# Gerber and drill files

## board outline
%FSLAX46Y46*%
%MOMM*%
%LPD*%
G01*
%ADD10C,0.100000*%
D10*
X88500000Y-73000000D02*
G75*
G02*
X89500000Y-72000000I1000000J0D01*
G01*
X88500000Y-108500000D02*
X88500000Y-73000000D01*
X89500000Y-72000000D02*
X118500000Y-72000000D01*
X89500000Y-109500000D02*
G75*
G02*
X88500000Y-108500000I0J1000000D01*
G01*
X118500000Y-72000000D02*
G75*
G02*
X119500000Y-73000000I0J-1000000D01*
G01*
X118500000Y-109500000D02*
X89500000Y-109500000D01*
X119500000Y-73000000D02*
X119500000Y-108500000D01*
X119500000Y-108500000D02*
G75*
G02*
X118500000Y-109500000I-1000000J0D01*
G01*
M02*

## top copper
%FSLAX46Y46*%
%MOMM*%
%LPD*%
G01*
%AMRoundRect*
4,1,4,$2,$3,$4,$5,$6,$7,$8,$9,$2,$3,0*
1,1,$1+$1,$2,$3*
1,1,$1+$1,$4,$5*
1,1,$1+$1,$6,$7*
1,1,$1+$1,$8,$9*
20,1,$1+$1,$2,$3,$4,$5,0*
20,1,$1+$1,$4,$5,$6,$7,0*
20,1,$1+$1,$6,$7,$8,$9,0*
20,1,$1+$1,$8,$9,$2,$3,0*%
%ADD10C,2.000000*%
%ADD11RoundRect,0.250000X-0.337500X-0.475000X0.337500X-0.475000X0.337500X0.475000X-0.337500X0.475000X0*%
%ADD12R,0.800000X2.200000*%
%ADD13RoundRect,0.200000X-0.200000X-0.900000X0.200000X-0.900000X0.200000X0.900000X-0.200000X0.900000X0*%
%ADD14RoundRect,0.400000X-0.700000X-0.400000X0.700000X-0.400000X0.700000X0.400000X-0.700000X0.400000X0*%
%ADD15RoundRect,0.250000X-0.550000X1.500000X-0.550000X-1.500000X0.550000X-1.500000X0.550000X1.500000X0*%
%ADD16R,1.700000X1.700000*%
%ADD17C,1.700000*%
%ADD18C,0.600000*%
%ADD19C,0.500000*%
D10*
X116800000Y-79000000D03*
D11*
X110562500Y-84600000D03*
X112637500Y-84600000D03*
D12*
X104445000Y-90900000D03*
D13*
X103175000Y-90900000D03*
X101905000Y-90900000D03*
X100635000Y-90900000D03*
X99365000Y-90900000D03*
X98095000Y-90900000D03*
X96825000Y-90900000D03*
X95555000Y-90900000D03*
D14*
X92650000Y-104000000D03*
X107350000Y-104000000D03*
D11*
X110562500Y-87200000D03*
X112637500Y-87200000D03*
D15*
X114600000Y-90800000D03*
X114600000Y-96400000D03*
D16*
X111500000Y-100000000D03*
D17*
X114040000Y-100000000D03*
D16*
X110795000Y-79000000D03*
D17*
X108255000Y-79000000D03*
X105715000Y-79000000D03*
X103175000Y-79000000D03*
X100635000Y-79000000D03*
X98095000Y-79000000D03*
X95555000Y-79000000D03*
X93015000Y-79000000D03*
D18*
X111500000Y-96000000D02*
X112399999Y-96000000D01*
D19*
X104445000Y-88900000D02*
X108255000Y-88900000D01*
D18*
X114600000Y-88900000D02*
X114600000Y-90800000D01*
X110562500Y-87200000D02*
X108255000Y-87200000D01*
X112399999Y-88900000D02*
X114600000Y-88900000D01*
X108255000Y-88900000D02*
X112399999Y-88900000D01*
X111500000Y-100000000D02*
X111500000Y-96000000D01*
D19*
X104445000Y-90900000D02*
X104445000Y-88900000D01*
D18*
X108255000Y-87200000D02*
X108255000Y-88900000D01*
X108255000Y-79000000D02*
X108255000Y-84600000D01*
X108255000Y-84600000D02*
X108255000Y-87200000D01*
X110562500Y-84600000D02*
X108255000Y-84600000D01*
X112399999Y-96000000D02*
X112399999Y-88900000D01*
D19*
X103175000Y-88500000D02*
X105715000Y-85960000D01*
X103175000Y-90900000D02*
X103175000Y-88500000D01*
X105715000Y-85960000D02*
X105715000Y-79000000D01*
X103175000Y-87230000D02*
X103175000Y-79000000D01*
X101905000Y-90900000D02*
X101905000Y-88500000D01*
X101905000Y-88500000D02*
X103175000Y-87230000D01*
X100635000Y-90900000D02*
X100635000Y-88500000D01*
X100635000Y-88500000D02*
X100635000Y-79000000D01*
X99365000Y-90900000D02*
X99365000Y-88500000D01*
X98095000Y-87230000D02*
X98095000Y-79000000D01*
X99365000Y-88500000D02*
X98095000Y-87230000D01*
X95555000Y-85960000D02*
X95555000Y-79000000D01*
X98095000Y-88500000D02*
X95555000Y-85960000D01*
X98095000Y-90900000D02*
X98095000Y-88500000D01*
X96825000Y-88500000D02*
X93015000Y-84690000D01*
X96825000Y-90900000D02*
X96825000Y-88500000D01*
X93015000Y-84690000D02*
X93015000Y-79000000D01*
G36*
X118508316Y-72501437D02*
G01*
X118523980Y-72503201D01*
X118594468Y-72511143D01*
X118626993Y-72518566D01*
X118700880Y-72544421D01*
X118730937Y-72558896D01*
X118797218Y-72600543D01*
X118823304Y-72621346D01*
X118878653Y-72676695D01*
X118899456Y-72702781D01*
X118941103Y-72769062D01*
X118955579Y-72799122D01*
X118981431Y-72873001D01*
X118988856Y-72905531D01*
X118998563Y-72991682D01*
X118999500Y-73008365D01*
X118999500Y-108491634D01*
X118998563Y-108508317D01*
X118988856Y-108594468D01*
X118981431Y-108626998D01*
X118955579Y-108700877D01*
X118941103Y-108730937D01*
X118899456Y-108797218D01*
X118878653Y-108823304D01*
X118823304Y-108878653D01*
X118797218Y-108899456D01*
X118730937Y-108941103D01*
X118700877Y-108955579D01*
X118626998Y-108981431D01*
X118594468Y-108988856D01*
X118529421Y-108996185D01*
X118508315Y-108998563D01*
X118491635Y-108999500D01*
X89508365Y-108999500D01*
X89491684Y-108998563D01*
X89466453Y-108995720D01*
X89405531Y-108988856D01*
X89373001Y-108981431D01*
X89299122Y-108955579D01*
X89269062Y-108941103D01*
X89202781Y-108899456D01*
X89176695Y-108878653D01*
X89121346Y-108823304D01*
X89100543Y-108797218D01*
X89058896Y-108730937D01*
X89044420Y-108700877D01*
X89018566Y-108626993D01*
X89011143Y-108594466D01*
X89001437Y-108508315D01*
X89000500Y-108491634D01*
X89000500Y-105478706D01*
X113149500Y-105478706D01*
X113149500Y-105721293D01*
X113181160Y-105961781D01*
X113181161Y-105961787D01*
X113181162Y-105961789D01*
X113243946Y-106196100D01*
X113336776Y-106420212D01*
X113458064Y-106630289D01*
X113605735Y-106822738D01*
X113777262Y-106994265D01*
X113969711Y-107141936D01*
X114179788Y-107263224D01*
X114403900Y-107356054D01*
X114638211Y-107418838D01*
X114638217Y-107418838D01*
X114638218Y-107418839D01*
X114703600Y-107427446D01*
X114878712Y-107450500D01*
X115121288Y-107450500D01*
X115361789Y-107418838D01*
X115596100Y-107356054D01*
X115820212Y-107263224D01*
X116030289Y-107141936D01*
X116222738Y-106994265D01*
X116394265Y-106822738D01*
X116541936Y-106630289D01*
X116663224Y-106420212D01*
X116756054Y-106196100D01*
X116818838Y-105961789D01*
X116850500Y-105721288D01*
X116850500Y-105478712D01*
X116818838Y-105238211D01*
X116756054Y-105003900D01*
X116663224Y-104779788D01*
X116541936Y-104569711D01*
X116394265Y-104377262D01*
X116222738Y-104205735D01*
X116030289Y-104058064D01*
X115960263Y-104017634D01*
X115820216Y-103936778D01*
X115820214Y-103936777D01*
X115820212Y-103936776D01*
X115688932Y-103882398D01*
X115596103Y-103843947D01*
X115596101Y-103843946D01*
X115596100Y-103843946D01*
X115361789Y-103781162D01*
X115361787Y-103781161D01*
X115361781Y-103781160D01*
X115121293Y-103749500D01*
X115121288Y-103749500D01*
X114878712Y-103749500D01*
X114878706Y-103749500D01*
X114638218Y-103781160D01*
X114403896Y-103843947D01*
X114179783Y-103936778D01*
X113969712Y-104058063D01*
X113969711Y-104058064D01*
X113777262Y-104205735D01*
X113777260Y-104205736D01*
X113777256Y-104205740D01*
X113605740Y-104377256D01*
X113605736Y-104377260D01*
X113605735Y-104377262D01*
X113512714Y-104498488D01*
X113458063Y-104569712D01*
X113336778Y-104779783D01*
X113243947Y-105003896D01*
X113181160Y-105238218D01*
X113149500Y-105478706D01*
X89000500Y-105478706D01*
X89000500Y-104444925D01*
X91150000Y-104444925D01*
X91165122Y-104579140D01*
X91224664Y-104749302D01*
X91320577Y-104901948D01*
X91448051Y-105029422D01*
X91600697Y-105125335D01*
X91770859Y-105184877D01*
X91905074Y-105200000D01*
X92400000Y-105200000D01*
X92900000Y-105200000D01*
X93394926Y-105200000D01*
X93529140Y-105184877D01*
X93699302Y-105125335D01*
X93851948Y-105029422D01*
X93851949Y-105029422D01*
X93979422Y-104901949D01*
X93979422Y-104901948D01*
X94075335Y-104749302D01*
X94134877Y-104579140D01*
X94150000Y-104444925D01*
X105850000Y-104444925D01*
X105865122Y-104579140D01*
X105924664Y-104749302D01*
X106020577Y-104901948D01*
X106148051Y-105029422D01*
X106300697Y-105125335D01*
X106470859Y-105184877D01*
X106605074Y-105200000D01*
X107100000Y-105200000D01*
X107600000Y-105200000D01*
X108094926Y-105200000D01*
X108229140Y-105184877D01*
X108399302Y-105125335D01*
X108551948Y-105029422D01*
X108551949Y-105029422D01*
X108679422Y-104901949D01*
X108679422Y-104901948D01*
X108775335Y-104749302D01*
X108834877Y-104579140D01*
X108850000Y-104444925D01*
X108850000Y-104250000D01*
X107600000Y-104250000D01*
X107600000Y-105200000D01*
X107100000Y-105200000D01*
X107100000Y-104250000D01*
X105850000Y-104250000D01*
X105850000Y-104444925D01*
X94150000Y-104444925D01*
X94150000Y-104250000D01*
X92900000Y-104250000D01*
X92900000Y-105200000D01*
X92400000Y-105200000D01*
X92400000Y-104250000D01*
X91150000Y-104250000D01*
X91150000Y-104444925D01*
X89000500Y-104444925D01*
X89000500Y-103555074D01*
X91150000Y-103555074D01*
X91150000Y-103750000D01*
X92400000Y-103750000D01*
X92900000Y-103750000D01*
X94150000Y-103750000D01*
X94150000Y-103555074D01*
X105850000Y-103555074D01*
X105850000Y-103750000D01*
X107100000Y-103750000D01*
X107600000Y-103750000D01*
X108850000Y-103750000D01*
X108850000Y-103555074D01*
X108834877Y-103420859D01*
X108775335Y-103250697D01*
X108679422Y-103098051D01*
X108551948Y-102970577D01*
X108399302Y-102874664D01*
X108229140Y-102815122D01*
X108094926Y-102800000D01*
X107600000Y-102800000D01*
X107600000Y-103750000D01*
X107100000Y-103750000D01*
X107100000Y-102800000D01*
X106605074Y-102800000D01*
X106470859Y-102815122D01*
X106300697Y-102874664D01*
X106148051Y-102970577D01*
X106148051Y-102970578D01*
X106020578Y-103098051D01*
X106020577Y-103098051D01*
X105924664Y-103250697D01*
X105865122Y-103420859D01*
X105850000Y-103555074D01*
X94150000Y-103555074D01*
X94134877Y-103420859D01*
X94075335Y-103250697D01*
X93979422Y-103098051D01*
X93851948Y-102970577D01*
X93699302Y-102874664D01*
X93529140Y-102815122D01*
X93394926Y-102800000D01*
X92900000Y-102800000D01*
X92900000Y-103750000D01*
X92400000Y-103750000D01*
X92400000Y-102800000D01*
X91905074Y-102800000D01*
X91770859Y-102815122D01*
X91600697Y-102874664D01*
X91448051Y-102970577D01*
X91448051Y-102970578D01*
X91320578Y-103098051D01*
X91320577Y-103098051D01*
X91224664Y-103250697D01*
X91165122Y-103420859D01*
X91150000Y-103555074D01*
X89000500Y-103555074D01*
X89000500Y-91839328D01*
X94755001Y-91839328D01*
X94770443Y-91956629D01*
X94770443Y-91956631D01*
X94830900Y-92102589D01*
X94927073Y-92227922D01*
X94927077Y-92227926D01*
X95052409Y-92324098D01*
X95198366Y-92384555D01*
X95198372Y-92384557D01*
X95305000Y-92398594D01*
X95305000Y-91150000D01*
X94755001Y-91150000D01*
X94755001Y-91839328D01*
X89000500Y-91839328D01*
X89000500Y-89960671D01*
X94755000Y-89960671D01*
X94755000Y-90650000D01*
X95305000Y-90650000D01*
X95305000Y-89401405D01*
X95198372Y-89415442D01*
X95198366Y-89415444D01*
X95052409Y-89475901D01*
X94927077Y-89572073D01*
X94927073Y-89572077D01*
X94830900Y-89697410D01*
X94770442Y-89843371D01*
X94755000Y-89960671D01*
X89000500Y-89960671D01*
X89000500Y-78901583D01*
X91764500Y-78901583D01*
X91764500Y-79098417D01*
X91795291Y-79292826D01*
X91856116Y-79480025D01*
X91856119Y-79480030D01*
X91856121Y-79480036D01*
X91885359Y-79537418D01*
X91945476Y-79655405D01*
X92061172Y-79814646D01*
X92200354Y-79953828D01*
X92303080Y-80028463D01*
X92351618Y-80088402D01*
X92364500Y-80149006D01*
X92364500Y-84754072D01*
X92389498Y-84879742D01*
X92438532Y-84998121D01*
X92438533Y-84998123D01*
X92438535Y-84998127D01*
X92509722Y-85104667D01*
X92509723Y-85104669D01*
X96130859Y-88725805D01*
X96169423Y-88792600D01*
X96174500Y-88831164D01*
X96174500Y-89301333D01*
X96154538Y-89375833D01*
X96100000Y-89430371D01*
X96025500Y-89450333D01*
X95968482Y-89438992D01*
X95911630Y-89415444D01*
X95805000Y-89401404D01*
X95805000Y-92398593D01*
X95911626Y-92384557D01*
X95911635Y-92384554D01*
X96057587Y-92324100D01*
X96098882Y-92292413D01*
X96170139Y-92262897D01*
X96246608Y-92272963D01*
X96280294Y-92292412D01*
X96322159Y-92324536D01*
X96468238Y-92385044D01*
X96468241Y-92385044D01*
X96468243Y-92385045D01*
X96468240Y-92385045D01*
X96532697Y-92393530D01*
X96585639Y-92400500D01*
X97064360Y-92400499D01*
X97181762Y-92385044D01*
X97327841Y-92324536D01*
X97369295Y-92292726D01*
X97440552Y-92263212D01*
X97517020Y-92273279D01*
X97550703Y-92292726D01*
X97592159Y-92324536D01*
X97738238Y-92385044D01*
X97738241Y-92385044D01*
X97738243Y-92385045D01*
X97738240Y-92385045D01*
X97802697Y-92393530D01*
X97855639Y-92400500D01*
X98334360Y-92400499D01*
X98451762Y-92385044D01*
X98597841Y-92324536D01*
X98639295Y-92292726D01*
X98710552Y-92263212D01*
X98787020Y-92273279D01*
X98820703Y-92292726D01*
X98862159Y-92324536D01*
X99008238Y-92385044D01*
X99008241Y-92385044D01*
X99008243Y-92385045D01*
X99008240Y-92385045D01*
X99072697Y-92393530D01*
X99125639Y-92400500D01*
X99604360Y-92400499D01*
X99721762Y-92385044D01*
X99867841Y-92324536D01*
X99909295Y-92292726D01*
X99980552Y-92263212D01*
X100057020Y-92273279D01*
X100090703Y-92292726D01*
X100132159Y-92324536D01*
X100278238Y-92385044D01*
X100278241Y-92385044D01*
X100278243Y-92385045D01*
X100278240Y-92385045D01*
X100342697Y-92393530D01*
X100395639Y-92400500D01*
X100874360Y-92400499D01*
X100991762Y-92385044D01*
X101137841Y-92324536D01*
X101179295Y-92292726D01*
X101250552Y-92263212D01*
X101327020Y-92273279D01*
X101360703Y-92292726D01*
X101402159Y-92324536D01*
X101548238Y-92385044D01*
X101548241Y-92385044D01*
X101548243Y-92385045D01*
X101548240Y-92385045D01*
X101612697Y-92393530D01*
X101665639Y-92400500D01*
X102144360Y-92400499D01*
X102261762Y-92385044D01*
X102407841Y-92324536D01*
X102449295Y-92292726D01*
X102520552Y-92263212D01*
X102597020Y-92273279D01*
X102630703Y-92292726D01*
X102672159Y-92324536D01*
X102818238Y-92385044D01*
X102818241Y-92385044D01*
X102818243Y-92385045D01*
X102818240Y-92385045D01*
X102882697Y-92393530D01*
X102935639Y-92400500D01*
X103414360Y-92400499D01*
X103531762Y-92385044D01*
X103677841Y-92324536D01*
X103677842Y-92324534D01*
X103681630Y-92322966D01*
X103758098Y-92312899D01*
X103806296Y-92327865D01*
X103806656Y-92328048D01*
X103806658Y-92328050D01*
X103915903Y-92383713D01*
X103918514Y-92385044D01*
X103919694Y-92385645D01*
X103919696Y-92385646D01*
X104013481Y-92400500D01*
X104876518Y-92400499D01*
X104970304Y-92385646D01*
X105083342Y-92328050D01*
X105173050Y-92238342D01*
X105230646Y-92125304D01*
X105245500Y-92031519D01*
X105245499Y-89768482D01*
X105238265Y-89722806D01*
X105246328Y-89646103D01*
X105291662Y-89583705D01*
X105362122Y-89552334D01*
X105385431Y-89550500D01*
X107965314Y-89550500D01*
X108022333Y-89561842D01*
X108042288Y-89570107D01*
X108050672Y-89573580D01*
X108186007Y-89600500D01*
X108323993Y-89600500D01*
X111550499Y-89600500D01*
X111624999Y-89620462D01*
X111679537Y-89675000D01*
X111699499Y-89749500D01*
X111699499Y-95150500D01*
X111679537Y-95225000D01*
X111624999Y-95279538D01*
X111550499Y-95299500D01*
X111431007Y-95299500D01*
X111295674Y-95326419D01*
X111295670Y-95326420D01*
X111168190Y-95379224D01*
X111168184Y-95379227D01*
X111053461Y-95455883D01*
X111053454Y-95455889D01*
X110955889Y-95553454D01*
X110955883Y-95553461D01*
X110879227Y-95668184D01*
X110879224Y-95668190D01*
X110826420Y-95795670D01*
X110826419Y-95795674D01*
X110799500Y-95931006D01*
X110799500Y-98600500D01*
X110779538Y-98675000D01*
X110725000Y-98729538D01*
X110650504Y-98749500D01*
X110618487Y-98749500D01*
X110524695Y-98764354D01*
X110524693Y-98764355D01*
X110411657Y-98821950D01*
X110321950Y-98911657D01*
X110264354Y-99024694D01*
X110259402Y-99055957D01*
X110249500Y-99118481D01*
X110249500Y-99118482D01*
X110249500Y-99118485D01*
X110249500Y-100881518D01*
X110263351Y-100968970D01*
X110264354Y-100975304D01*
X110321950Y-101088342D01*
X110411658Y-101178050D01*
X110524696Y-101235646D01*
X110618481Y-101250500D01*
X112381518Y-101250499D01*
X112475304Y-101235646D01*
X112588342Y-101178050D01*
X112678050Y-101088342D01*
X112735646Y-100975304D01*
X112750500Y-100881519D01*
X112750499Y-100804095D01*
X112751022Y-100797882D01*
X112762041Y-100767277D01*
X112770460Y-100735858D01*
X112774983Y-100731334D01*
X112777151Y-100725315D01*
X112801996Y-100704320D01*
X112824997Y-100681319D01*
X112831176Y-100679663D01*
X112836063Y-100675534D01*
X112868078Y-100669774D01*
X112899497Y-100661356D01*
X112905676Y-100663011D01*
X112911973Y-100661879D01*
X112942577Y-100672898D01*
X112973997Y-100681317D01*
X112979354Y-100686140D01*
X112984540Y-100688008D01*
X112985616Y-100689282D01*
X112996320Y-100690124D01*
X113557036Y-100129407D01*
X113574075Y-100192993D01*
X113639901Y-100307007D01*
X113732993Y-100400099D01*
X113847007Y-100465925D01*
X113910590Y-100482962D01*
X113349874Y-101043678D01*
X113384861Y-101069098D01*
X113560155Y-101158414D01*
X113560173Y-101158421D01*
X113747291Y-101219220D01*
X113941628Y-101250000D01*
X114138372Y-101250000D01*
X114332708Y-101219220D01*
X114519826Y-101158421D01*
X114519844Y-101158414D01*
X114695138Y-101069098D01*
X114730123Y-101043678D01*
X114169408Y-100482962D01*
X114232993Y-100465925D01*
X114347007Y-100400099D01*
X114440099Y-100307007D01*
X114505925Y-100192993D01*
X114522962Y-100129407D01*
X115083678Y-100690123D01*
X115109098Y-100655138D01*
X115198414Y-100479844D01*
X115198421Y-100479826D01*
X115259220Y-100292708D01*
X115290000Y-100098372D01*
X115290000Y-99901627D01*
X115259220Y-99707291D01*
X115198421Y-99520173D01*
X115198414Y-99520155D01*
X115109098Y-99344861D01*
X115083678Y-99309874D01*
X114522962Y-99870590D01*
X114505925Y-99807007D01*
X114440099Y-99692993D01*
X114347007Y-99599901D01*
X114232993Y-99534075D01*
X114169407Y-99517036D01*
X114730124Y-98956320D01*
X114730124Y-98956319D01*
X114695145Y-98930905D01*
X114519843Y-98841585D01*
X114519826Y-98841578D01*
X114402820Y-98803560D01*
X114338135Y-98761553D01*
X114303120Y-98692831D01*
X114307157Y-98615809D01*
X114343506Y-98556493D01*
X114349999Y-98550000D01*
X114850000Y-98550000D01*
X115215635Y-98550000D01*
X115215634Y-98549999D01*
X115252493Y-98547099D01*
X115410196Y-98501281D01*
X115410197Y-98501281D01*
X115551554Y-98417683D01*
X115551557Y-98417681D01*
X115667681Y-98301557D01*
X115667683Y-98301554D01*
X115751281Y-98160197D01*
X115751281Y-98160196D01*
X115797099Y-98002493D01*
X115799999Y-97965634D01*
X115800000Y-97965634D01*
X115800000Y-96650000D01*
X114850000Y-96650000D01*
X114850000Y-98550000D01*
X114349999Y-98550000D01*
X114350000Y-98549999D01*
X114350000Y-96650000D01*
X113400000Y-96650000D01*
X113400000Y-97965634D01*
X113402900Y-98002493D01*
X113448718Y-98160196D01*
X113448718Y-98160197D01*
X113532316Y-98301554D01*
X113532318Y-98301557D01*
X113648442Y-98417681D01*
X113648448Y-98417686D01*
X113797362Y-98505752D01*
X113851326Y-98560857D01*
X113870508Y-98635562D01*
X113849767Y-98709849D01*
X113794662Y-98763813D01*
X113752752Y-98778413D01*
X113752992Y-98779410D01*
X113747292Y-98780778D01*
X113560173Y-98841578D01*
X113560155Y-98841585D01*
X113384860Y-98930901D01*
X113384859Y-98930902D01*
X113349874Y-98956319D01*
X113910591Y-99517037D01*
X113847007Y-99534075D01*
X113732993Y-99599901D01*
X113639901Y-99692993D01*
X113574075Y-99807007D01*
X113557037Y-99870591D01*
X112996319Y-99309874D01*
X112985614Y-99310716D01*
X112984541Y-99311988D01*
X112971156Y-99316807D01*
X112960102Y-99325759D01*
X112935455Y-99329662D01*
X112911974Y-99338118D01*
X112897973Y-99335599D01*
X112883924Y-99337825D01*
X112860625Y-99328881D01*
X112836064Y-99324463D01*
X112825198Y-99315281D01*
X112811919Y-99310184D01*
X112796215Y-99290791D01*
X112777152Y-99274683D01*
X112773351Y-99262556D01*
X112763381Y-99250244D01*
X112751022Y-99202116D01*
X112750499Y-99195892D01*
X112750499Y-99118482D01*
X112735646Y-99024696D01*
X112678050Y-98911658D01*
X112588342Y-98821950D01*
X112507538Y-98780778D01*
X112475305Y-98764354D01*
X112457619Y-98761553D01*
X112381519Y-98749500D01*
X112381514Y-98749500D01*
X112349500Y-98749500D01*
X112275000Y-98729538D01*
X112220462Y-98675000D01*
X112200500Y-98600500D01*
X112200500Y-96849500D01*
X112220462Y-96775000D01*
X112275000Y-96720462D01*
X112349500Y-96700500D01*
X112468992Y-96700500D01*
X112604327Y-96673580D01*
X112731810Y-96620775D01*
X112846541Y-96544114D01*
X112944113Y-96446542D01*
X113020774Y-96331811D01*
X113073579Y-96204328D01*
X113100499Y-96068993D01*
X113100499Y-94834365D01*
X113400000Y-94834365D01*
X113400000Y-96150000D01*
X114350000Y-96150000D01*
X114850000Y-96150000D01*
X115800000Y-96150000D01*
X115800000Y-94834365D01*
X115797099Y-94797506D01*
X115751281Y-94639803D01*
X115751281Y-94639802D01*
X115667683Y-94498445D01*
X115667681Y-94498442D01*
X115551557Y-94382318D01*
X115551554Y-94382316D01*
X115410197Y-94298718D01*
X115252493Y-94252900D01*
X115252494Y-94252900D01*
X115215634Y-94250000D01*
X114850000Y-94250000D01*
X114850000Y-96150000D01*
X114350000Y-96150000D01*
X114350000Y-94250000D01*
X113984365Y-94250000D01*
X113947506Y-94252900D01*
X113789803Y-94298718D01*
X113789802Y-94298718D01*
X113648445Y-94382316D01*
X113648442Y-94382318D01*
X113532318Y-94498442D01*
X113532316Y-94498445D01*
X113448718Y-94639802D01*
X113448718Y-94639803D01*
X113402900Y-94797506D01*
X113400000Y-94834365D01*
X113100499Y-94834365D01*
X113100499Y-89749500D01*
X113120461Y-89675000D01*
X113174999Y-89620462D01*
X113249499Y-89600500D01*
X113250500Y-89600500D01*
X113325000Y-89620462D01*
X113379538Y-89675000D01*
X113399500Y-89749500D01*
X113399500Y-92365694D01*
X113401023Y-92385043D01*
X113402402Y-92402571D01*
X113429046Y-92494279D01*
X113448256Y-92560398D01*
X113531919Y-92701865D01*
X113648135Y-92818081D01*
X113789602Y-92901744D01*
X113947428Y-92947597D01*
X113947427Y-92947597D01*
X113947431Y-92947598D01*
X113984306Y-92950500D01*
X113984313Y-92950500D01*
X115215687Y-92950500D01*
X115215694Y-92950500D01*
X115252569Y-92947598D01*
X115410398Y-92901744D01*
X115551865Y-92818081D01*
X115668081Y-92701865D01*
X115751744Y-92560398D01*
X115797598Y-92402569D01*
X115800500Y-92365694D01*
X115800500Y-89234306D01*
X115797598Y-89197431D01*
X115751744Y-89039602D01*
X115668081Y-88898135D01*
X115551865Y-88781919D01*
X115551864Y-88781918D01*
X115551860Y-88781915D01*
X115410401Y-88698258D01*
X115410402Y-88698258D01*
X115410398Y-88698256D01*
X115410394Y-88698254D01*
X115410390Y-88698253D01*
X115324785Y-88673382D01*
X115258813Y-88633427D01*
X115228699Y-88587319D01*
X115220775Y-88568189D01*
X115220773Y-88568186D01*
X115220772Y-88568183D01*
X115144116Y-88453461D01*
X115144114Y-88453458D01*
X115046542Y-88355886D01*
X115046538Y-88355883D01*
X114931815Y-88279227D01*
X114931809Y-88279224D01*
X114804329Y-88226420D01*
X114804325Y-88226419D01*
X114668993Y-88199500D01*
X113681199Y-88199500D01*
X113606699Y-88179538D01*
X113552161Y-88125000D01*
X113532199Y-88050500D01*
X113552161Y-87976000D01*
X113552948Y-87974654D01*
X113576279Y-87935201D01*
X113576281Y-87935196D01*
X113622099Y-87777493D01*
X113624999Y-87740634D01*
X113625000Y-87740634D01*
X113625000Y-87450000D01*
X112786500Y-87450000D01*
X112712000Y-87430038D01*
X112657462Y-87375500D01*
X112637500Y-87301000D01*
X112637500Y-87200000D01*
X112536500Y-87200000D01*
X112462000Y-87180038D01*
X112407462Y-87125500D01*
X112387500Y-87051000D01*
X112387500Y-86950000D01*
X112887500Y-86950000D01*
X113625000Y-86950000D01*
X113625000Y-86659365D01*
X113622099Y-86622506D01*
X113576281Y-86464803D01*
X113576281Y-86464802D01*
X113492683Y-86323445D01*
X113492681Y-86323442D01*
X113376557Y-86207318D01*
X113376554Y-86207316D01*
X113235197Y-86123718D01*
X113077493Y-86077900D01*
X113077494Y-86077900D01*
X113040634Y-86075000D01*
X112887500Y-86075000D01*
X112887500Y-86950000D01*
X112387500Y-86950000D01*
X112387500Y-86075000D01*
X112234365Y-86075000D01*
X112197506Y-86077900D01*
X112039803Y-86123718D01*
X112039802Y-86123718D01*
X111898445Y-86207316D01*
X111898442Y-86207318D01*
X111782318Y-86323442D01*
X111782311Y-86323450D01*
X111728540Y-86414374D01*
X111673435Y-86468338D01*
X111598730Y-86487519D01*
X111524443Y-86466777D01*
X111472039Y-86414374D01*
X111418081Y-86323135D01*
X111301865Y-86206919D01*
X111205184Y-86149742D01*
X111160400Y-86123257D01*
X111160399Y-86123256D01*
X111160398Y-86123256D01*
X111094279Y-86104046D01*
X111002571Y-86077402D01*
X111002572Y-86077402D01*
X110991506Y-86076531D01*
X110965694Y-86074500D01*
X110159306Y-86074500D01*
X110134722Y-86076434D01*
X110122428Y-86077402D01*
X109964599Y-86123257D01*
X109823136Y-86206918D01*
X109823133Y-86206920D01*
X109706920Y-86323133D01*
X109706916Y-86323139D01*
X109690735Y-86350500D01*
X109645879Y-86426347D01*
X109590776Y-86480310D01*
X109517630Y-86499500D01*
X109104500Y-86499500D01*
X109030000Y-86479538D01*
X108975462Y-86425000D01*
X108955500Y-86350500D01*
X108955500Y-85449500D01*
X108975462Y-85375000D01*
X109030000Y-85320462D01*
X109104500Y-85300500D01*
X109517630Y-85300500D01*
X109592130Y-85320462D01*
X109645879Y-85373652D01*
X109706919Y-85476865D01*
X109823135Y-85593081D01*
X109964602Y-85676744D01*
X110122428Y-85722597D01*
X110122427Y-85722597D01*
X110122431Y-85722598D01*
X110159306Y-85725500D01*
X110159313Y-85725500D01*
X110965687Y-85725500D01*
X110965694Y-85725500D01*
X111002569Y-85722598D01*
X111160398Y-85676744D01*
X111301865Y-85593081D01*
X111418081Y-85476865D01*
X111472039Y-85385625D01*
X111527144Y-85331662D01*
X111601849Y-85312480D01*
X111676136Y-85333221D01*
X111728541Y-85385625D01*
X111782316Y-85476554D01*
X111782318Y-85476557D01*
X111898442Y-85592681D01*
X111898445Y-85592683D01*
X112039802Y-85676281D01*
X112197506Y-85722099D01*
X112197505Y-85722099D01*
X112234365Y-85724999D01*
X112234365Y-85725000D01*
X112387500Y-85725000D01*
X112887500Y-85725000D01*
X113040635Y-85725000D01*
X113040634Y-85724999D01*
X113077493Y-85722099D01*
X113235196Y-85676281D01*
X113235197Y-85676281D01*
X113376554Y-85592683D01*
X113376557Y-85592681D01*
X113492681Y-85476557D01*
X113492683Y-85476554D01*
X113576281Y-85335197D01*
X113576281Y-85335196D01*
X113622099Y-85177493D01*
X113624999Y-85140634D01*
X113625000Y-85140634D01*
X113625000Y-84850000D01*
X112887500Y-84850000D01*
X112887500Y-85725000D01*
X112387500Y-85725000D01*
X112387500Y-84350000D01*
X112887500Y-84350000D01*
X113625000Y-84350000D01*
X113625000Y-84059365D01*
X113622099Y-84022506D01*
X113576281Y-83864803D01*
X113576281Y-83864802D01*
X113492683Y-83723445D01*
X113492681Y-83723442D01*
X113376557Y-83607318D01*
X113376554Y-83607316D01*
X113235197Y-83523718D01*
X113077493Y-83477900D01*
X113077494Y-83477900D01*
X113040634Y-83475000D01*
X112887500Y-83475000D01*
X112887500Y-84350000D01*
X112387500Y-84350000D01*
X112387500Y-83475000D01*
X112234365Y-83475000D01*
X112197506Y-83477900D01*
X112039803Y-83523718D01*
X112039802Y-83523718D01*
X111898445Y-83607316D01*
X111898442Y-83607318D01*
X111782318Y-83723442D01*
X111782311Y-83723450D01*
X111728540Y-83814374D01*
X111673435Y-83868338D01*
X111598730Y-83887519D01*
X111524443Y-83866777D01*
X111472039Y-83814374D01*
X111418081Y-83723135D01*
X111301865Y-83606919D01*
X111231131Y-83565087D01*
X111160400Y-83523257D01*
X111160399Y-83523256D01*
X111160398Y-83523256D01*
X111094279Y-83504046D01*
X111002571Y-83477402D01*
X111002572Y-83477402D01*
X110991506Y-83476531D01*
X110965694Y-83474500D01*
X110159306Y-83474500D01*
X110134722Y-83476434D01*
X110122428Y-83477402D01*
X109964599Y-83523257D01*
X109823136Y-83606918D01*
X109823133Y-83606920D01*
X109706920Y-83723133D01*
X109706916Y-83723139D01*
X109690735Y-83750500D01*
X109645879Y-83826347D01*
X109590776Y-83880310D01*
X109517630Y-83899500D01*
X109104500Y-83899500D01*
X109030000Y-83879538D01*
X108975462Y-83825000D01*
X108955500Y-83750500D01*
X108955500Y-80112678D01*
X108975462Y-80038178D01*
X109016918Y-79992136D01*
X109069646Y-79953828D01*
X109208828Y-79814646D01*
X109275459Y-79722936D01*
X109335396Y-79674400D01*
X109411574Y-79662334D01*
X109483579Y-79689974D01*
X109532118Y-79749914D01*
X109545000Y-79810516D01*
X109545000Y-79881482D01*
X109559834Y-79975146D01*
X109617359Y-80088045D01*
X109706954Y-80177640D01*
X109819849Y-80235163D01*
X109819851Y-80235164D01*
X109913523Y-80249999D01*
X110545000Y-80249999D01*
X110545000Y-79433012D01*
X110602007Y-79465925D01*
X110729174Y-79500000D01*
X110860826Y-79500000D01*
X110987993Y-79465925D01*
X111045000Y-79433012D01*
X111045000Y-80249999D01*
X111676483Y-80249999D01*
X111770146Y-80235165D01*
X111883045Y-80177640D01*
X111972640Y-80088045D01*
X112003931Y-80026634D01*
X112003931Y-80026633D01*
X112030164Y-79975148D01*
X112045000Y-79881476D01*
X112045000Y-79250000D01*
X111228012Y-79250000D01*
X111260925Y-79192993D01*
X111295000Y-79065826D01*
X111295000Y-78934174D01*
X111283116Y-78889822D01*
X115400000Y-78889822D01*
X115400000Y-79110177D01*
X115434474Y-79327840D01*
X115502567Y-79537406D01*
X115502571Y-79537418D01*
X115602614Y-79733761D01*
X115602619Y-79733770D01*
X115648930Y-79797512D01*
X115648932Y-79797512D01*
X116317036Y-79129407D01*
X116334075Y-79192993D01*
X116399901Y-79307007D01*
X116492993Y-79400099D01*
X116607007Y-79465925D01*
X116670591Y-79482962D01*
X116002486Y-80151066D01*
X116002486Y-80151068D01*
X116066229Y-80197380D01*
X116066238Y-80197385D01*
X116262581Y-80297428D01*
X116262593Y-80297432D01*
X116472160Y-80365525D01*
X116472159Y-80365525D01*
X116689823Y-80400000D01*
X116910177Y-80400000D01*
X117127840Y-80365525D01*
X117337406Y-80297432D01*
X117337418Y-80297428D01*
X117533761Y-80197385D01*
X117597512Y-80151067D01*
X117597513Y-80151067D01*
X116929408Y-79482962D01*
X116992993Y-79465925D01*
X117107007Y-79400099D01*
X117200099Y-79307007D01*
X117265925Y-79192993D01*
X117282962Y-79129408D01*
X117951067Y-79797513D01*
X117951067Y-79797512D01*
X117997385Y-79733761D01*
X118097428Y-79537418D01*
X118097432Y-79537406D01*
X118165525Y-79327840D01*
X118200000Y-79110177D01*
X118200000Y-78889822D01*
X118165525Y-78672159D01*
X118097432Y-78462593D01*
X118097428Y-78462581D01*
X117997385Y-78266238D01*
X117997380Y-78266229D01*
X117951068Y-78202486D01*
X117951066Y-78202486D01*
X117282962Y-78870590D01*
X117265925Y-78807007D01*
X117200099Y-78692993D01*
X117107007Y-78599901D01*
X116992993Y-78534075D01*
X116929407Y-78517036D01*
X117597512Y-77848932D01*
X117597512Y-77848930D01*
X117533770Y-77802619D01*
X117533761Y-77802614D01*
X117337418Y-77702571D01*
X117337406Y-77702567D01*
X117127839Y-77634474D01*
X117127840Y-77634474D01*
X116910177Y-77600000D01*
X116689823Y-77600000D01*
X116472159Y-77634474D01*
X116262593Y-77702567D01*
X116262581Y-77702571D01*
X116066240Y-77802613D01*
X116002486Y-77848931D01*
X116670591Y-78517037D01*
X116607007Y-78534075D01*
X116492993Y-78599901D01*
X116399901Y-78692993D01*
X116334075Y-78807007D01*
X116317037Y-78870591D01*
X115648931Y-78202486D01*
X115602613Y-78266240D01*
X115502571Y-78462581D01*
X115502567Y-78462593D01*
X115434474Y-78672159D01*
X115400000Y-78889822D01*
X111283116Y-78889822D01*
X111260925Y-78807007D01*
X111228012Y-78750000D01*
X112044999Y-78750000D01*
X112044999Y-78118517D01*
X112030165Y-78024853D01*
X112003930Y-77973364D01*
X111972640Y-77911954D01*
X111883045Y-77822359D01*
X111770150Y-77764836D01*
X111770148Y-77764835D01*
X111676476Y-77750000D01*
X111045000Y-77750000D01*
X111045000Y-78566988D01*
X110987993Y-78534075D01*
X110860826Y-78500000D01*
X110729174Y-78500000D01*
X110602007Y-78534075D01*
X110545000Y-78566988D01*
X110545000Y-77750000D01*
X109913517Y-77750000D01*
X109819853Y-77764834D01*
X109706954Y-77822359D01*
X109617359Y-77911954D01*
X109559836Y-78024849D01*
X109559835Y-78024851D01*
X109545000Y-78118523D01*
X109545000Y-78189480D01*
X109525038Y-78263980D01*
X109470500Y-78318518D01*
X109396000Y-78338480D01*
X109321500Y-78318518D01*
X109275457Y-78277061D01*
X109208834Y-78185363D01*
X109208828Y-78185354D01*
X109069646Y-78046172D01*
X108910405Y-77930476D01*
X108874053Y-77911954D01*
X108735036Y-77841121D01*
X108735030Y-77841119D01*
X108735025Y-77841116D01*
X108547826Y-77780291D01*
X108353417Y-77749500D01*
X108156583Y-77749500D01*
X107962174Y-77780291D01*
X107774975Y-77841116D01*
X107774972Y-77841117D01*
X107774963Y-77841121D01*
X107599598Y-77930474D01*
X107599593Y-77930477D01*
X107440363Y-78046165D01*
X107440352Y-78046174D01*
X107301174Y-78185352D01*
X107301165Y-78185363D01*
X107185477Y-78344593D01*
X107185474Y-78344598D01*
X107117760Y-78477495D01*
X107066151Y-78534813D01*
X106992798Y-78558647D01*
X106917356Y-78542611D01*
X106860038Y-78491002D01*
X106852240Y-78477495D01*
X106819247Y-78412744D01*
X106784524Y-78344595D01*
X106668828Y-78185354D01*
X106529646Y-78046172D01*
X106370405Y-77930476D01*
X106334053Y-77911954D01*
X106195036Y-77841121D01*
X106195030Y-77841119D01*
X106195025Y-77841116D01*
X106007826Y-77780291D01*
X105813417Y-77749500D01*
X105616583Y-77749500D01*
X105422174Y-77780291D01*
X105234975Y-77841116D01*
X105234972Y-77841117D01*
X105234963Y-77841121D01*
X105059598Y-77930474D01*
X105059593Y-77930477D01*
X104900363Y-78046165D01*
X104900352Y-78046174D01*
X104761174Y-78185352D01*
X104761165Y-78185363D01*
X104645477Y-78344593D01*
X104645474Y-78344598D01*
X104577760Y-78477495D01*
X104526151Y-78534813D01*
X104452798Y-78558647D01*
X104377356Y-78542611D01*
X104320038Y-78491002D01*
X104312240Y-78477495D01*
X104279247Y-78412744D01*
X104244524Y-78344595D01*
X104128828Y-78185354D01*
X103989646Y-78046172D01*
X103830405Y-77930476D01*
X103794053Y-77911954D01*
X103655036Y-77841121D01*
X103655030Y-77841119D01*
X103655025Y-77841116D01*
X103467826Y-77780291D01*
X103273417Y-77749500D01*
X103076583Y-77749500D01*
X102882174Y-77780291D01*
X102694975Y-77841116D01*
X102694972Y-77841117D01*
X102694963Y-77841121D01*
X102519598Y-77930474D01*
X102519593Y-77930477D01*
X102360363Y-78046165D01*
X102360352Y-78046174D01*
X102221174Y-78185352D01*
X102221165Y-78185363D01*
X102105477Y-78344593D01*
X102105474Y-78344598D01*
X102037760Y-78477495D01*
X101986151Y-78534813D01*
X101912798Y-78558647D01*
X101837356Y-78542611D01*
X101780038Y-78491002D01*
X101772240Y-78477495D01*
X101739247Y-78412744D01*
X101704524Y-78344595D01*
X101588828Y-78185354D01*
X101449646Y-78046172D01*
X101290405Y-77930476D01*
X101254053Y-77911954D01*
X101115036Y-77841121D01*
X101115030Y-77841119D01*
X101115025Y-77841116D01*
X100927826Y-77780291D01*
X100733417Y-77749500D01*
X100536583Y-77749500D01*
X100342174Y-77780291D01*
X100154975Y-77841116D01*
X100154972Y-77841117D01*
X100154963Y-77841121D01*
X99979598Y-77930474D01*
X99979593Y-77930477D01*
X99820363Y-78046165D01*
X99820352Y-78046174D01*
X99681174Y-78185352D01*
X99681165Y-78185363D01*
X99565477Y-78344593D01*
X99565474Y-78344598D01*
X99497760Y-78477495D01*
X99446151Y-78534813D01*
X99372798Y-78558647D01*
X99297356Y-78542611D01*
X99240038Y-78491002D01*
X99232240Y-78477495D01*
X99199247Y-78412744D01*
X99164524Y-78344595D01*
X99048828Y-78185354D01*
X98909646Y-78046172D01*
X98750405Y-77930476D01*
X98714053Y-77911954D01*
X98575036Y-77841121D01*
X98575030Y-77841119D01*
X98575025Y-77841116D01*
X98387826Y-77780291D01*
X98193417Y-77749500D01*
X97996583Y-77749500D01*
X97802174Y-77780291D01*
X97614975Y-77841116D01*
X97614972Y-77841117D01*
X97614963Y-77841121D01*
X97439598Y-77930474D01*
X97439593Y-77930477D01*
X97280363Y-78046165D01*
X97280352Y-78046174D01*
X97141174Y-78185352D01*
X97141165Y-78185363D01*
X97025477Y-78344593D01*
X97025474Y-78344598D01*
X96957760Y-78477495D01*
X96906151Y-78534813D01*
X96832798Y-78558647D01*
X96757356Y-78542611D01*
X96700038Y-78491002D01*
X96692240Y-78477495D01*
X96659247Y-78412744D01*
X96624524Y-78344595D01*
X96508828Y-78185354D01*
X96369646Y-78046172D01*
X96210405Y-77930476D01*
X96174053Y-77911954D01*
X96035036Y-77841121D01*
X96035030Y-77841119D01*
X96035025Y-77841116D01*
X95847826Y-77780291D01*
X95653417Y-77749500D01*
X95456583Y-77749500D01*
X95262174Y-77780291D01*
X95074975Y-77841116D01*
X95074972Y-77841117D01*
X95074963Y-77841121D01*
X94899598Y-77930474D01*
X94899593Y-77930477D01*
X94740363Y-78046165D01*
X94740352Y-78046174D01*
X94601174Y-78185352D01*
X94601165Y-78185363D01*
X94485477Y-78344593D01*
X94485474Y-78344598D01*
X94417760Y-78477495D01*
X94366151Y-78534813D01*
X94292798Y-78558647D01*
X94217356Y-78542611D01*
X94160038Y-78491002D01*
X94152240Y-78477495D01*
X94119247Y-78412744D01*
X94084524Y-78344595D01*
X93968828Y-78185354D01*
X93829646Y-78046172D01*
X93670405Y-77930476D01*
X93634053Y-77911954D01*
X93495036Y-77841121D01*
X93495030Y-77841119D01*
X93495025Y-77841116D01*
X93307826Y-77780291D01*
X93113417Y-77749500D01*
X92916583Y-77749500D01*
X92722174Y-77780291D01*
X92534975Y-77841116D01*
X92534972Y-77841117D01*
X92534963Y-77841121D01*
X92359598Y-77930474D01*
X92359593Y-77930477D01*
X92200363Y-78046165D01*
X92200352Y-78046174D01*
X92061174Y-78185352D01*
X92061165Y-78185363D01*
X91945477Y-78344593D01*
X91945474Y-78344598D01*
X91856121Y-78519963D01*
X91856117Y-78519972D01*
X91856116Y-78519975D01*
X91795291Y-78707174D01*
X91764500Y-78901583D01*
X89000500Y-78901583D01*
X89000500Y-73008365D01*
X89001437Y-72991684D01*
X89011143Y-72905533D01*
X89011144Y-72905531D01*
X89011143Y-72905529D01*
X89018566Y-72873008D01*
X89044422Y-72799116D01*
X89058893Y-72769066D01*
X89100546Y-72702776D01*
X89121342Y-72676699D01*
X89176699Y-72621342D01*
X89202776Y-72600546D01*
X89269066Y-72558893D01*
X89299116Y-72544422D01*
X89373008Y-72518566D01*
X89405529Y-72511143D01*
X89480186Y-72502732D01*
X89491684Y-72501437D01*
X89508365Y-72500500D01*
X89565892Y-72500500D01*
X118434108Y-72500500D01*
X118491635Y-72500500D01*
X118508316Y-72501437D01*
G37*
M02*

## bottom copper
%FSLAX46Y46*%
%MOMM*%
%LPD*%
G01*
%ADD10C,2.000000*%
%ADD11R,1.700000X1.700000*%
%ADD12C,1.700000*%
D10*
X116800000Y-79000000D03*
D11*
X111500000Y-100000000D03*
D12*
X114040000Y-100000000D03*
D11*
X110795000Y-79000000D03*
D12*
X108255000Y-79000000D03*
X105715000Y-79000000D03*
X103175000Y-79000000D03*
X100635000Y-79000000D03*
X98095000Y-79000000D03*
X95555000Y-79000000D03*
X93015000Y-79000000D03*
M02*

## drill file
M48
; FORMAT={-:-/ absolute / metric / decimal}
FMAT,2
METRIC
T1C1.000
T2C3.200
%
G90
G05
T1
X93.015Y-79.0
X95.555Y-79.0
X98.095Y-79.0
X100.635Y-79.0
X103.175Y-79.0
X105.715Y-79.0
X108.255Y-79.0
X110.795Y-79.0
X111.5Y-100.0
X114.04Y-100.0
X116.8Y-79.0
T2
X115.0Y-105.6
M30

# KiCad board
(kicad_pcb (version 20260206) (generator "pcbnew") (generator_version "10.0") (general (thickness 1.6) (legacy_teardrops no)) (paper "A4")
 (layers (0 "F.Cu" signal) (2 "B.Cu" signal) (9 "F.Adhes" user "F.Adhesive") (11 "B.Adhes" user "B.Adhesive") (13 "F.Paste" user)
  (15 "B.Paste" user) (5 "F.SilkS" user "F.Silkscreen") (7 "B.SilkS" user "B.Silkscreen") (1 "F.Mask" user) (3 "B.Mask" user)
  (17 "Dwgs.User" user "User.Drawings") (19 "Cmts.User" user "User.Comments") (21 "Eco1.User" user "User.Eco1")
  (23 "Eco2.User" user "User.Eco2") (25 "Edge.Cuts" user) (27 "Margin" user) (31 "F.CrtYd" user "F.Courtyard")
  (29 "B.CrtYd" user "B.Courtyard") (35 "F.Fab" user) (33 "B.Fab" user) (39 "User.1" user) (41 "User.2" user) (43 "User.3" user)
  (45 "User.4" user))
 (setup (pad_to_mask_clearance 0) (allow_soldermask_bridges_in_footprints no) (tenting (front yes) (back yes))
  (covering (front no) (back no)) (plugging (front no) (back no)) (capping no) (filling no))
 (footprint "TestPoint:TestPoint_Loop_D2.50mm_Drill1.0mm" (layer "F.Cu") (at 116.8 79)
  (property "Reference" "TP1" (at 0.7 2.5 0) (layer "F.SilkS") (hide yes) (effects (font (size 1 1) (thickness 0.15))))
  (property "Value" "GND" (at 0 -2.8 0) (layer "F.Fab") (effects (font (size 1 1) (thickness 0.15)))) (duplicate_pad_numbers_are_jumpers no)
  (pad "1" thru_hole circle (at 0 0) (size 2 2) (drill 1) (layers "*.Cu" "*.Mask") (remove_unused_layers no) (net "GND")))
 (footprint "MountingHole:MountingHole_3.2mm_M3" (layer "F.Cu") (at 115 105.6)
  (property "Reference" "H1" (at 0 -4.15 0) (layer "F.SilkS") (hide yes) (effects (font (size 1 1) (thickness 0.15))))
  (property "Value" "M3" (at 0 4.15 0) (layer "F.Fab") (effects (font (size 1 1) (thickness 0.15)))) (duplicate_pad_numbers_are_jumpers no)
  (pad "" np_thru_hole circle (at 0 0) (size 3.2 3.2) (drill 3.2) (layers "*.Cu" "*.Mask")))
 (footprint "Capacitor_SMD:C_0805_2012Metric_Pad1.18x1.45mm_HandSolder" (layer "F.Cu") (at 111.6 84.6)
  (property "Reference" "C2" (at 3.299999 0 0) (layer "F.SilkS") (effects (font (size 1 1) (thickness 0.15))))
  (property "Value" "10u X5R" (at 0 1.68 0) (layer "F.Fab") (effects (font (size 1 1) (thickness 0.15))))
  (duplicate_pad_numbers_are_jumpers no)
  (pad "1" smd roundrect (at -1.0375 0) (size 1.175 1.45) (layers "F.Cu" "F.Mask" "F.Paste") (roundrect_rratio 0.212766) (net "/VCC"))
  (pad "2" smd roundrect (at 1.0375 0) (size 1.175 1.45) (layers "F.Cu" "F.Mask" "F.Paste") (roundrect_rratio 0.212766) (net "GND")))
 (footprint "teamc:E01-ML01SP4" (layer "F.Cu") (at 100 100)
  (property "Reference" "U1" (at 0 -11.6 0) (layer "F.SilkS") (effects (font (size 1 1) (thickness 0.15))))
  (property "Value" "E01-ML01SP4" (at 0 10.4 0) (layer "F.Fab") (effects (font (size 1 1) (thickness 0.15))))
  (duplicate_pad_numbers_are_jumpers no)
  (pad "1" smd rect (at 4.445 -9.1) (size 0.8 2.2) (layers "F.Cu" "F.Mask" "F.Paste") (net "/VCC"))
  (pad "2" smd roundrect (at 3.175 -9.1) (size 0.8 2.2) (layers "F.Cu" "F.Mask" "F.Paste") (roundrect_rratio 0.25) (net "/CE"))
  (pad "3" smd roundrect (at 1.905 -9.1) (size 0.8 2.2) (layers "F.Cu" "F.Mask" "F.Paste") (roundrect_rratio 0.25) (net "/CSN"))
  (pad "4" smd roundrect (at 0.635 -9.1) (size 0.8 2.2) (layers "F.Cu" "F.Mask" "F.Paste") (roundrect_rratio 0.25) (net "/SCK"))
  (pad "5" smd roundrect (at -0.635 -9.1) (size 0.8 2.2) (layers "F.Cu" "F.Mask" "F.Paste") (roundrect_rratio 0.25) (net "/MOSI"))
  (pad "6" smd roundrect (at -1.905 -9.1) (size 0.8 2.2) (layers "F.Cu" "F.Mask" "F.Paste") (roundrect_rratio 0.25) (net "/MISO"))
  (pad "7" smd roundrect (at -3.175 -9.1) (size 0.8 2.2) (layers "F.Cu" "F.Mask" "F.Paste") (roundrect_rratio 0.25) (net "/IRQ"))
  (pad "8" smd roundrect (at -4.445 -9.1) (size 0.8 2.2) (layers "F.Cu" "F.Mask" "F.Paste") (roundrect_rratio 0.25) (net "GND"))
  (pad "9" smd roundrect (at -7.35 4) (size 2.2 1.6) (layers "F.Cu" "F.Mask" "F.Paste") (roundrect_rratio 0.25) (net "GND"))
  (pad "10" smd roundrect (at 7.35 4) (size 2.2 1.6) (layers "F.Cu" "F.Mask" "F.Paste") (roundrect_rratio 0.25) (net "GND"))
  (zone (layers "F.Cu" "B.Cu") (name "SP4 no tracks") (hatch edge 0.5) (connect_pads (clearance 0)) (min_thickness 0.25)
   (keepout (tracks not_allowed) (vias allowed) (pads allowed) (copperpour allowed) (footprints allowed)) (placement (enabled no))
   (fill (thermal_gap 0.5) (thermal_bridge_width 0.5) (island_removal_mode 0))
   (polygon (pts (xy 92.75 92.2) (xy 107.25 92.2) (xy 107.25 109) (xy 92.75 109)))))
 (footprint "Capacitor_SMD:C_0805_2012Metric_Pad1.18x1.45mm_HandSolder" (layer "F.Cu") (at 111.6 87.2)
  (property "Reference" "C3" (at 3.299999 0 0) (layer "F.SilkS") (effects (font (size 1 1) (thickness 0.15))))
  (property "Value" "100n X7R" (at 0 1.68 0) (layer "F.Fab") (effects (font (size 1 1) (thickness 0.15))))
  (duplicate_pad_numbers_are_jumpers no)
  (pad "1" smd roundrect (at -1.0375 0) (size 1.175 1.45) (layers "F.Cu" "F.Mask" "F.Paste") (roundrect_rratio 0.212766) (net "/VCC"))
  (pad "2" smd roundrect (at 1.0375 0) (size 1.175 1.45) (layers "F.Cu" "F.Mask" "F.Paste") (roundrect_rratio 0.212766) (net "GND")))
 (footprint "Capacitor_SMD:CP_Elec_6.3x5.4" (layer "F.Cu") (at 114.6 93.6 -90)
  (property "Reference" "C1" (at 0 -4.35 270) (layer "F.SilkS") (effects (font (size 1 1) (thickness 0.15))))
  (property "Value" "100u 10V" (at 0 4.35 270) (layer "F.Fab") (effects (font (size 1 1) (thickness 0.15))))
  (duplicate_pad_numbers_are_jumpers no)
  (pad "1" smd roundrect (at -2.8 0 270) (size 3.5 1.6) (layers "F.Cu" "F.Mask" "F.Paste") (roundrect_rratio 0.15625) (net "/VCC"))
  (pad "2" smd roundrect (at 2.8 0 270) (size 3.5 1.6) (layers "F.Cu" "F.Mask" "F.Paste") (roundrect_rratio 0.15625) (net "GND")))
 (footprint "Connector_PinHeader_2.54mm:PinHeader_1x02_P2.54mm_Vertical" (layer "B.Cu") (at 111.5 100 -90)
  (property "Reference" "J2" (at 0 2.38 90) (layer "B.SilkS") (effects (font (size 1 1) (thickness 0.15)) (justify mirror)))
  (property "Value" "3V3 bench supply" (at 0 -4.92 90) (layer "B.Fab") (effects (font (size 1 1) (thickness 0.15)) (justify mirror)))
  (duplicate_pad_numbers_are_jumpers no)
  (pad "1" thru_hole rect (at 0 0 270) (size 1.7 1.7) (drill 1) (layers "*.Cu" "*.Mask") (remove_unused_layers no) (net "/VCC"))
  (pad "2" thru_hole circle (at 0 -2.54 270) (size 1.7 1.7) (drill 1) (layers "*.Cu" "*.Mask") (remove_unused_layers no) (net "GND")))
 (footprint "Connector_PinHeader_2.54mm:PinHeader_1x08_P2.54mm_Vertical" (layer "B.Cu") (at 110.795 79 90)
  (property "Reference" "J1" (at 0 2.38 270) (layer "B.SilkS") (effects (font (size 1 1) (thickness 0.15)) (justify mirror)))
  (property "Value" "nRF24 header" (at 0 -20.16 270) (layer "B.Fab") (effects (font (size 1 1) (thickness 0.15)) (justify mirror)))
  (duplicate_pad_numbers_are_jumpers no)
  (pad "1" thru_hole rect (at 0 0 90) (size 1.7 1.7) (drill 1) (layers "*.Cu" "*.Mask") (remove_unused_layers no) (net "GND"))
  (pad "2" thru_hole circle (at 0 -2.54 90) (size 1.7 1.7) (drill 1) (layers "*.Cu" "*.Mask") (remove_unused_layers no) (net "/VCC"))
  (pad "3" thru_hole circle (at 0 -5.08 90) (size 1.7 1.7) (drill 1) (layers "*.Cu" "*.Mask") (remove_unused_layers no) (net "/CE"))
  (pad "4" thru_hole circle (at 0 -7.62 90) (size 1.7 1.7) (drill 1) (layers "*.Cu" "*.Mask") (remove_unused_layers no) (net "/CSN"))
  (pad "5" thru_hole circle (at 0 -10.16 90) (size 1.7 1.7) (drill 1) (layers "*.Cu" "*.Mask") (remove_unused_layers no) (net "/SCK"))
  (pad "6" thru_hole circle (at 0 -12.7 90) (size 1.7 1.7) (drill 1) (layers "*.Cu" "*.Mask") (remove_unused_layers no) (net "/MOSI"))
  (pad "7" thru_hole circle (at 0 -15.24 90) (size 1.7 1.7) (drill 1) (layers "*.Cu" "*.Mask") (remove_unused_layers no) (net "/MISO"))
  (pad "8" thru_hole circle (at 0 -17.78 90) (size 1.7 1.7) (drill 1) (layers "*.Cu" "*.Mask") (remove_unused_layers no) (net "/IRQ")))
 (gr_arc (start 88.5 73) (mid 88.792893 72.292893) (end 89.5 72) (stroke (width 0.1) (type default)) (layer "Edge.Cuts"))
 (gr_line (start 88.5 108.5) (end 88.5 73) (stroke (width 0.1) (type default)) (layer "Edge.Cuts"))
 (gr_line (start 89.5 72) (end 118.5 72) (stroke (width 0.1) (type default)) (layer "Edge.Cuts"))
 (gr_arc (start 89.5 109.5) (mid 88.792893 109.207107) (end 88.5 108.5) (stroke (width 0.1) (type default)) (layer "Edge.Cuts"))
 (gr_arc (start 118.5 72) (mid 119.207107 72.292893) (end 119.5 73) (stroke (width 0.1) (type default)) (layer "Edge.Cuts"))
 (gr_line (start 118.5 109.5) (end 89.5 109.5) (stroke (width 0.1) (type default)) (layer "Edge.Cuts"))
 (gr_line (start 119.5 73) (end 119.5 108.5) (stroke (width 0.1) (type default)) (layer "Edge.Cuts"))
 (gr_arc (start 119.5 108.5) (mid 119.207107 109.207107) (end 118.5 109.5) (stroke (width 0.1) (type default)) (layer "Edge.Cuts"))
 (segment (start 111.5 96) (end 112.399999 96) (width 0.6) (layer "F.Cu") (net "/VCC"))
 (segment (start 104.445 88.9) (end 108.255 88.9) (width 0.5) (layer "F.Cu") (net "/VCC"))
 (segment (start 114.6 88.9) (end 114.6 90.8) (width 0.6) (layer "F.Cu") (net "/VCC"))
 (segment (start 110.5625 87.2) (end 108.255 87.2) (width 0.6) (layer "F.Cu") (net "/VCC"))
 (segment (start 112.399999 88.9) (end 114.6 88.9) (width 0.6) (layer "F.Cu") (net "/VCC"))
 (segment (start 108.255 88.9) (end 112.399999 88.9) (width 0.6) (layer "F.Cu") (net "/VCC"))
 (segment (start 111.5 100) (end 111.5 96) (width 0.6) (layer "F.Cu") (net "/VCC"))
 (segment (start 104.445 90.9) (end 104.445 88.9) (width 0.5) (layer "F.Cu") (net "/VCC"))
 (segment (start 108.255 87.2) (end 108.255 88.9) (width 0.6) (layer "F.Cu") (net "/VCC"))
 (segment (start 108.255 79) (end 108.255 84.6) (width 0.6) (layer "F.Cu") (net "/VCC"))
 (segment (start 108.255 84.6) (end 108.255 87.2) (width 0.6) (layer "F.Cu") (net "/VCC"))
 (segment (start 110.5625 84.6) (end 108.255 84.6) (width 0.6) (layer "F.Cu") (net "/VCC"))
 (segment (start 112.399999 96) (end 112.399999 88.9) (width 0.6) (layer "F.Cu") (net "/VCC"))
 (segment (start 103.175 88.5) (end 105.715 85.96) (width 0.5) (layer "F.Cu") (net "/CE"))
 (segment (start 103.175 90.9) (end 103.175 88.5) (width 0.5) (layer "F.Cu") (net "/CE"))
 (segment (start 105.715 85.96) (end 105.715 79) (width 0.5) (layer "F.Cu") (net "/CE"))
 (segment (start 103.175 87.23) (end 103.175 79) (width 0.5) (layer "F.Cu") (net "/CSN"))
 (segment (start 101.905 90.9) (end 101.905 88.5) (width 0.5) (layer "F.Cu") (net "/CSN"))
 (segment (start 101.905 88.5) (end 103.175 87.23) (width 0.5) (layer "F.Cu") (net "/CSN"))
 (segment (start 100.635 90.9) (end 100.635 88.5) (width 0.5) (layer "F.Cu") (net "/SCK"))
 (segment (start 100.635 88.5) (end 100.635 79) (width 0.5) (layer "F.Cu") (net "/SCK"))
 (segment (start 99.365 90.9) (end 99.365 88.5) (width 0.5) (layer "F.Cu") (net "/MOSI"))
 (segment (start 98.095 87.23) (end 98.095 79) (width 0.5) (layer "F.Cu") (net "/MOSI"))
 (segment (start 99.365 88.5) (end 98.095 87.23) (width 0.5) (layer "F.Cu") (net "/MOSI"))
 (segment (start 95.555 85.96) (end 95.555 79) (width 0.5) (layer "F.Cu") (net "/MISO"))
 (segment (start 98.095 88.5) (end 95.555 85.96) (width 0.5) (layer "F.Cu") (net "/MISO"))
 (segment (start 98.095 90.9) (end 98.095 88.5) (width 0.5) (layer "F.Cu") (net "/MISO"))
 (segment (start 96.825 88.5) (end 93.015 84.69) (width 0.5) (layer "F.Cu") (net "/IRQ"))
 (segment (start 96.825 90.9) (end 96.825 88.5) (width 0.5) (layer "F.Cu") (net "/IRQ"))
 (segment (start 93.015 84.69) (end 93.015 79) (width 0.5) (layer "F.Cu") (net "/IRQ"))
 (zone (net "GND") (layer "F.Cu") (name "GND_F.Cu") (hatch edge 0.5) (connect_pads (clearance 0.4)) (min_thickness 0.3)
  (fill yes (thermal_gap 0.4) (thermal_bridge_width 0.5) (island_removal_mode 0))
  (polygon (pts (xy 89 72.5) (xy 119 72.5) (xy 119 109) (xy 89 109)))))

